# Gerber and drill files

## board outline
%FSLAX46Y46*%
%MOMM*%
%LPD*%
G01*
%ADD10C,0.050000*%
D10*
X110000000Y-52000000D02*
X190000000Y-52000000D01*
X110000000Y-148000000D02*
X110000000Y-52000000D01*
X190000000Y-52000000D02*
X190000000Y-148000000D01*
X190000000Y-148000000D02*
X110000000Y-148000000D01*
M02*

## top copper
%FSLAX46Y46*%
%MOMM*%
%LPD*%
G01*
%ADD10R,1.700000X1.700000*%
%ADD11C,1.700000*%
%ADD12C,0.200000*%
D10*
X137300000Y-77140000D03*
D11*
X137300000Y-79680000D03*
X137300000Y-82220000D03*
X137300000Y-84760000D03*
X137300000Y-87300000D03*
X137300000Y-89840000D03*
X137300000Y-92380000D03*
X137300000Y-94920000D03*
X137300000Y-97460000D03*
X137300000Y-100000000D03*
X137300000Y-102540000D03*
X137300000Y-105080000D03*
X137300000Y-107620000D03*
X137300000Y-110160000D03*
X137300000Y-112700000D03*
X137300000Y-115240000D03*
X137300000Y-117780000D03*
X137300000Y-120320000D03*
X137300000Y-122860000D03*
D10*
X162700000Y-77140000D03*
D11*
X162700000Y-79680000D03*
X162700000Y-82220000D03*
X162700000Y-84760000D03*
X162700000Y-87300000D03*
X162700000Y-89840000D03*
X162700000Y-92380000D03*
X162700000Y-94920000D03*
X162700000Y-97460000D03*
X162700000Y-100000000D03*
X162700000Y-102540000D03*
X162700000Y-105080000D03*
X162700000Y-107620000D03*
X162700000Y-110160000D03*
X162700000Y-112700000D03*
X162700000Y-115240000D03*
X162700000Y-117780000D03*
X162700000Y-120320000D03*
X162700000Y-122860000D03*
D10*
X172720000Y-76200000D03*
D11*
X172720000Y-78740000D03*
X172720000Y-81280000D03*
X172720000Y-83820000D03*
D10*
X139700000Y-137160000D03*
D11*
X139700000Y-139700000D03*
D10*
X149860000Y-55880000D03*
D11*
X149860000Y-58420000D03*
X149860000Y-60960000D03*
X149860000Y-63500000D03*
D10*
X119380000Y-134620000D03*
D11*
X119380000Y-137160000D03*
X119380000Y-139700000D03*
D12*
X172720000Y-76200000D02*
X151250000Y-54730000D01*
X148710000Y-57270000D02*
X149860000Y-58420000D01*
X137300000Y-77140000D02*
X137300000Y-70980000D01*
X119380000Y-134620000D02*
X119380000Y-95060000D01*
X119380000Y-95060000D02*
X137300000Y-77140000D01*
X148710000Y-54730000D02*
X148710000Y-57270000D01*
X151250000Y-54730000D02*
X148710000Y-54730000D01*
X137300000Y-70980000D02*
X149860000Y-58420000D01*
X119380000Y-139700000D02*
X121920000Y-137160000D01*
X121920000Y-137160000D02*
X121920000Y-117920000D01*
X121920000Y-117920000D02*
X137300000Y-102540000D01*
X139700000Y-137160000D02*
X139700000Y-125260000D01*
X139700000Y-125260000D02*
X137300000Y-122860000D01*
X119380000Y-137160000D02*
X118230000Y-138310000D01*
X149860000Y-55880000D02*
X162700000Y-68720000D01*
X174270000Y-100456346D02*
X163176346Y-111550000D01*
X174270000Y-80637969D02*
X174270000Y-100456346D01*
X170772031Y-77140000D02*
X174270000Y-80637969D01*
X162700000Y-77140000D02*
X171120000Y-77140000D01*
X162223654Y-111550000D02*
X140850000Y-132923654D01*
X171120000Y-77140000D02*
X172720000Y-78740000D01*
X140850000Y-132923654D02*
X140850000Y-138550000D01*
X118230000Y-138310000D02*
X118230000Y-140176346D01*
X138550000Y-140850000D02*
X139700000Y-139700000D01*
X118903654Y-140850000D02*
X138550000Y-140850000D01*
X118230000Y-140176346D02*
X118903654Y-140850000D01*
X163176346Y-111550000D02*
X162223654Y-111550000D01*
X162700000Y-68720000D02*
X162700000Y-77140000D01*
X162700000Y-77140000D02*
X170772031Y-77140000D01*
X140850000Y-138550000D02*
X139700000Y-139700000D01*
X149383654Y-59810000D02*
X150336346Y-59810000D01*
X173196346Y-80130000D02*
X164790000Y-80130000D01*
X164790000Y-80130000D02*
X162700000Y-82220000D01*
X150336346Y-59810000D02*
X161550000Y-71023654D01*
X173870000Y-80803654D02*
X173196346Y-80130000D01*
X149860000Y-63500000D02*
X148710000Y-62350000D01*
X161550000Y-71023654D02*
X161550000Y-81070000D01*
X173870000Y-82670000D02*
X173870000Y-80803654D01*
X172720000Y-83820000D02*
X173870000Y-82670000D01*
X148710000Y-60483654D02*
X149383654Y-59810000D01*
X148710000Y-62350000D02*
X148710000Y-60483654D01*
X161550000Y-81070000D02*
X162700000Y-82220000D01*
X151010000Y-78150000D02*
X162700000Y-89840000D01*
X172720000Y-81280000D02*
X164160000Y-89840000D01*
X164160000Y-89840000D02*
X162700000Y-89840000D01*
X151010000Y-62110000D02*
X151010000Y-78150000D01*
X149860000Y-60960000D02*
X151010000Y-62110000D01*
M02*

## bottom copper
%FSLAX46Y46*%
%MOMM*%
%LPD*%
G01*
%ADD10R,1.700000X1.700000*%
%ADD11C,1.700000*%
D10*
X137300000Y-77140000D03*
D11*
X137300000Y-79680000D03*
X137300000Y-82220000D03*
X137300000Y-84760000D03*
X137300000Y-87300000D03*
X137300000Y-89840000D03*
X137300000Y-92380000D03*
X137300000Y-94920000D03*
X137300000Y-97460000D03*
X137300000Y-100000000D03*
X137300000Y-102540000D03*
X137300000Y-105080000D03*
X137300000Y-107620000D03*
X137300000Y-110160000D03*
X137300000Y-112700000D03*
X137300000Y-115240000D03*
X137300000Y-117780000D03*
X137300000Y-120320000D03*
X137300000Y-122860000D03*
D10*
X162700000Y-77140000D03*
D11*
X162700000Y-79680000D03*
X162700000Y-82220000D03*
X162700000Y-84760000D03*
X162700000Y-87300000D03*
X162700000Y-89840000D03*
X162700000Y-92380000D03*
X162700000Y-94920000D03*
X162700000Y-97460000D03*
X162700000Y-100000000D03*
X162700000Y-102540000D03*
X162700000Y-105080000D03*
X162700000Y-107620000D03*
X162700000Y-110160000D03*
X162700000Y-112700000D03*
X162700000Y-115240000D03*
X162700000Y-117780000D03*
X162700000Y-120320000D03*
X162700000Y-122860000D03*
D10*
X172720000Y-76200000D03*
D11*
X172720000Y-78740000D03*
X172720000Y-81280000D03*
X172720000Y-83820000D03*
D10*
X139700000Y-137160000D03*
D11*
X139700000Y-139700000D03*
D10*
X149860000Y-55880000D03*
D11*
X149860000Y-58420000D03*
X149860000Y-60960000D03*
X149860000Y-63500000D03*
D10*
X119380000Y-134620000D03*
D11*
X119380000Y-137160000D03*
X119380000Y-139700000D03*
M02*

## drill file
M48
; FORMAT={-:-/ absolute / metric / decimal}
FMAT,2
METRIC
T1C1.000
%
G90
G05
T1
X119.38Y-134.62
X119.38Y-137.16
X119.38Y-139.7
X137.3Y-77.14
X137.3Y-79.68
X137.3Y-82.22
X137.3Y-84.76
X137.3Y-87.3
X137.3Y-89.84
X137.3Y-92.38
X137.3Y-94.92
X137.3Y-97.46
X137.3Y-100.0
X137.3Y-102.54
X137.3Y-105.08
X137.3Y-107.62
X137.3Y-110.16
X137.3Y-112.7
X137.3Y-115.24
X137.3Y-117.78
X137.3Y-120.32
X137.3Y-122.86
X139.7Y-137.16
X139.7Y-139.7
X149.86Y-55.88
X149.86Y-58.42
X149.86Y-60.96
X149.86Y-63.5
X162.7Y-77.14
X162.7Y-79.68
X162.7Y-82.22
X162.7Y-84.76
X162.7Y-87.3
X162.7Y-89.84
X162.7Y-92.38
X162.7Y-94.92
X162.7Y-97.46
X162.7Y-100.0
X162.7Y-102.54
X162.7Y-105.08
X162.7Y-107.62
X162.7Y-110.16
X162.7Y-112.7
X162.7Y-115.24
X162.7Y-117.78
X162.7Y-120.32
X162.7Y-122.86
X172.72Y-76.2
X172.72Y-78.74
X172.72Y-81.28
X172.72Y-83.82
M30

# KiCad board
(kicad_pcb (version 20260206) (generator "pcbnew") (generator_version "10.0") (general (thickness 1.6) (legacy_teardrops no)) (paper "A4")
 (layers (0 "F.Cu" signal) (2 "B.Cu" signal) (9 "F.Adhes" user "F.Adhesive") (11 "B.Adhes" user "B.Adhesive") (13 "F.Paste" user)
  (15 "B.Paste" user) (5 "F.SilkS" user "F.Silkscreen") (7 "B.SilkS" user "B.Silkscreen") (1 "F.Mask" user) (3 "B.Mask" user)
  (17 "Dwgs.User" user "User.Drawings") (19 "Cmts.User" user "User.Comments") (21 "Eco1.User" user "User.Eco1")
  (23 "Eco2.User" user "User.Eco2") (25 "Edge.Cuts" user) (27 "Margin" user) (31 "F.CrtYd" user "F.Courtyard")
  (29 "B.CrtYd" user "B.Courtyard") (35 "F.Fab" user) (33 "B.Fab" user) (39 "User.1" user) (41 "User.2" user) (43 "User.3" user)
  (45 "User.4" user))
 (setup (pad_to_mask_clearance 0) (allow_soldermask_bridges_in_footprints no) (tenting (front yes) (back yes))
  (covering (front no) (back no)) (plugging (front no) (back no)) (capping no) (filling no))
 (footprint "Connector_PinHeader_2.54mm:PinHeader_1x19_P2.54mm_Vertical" (layer "F.Cu") (at 137.3 77.14)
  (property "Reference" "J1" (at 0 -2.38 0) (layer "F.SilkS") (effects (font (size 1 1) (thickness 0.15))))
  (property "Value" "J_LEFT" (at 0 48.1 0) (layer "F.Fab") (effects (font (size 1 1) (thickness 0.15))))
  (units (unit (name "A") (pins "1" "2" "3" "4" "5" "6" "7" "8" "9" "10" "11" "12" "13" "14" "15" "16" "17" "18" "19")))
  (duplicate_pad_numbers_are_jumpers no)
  (pad "1" thru_hole rect (at 0 0) (size 1.7 1.7) (drill 1) (layers "*.Cu" "*.Mask") (remove_unused_layers no) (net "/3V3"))
  (pad "2" thru_hole circle (at 0 2.54) (size 1.7 1.7) (drill 1) (layers "*.Cu" "*.Mask") (remove_unused_layers no)
   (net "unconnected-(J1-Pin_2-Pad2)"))
  (pad "3" thru_hole circle (at 0 5.08) (size 1.7 1.7) (drill 1) (layers "*.Cu" "*.Mask") (remove_unused_layers no)
   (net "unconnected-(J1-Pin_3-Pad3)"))
  (pad "4" thru_hole circle (at 0 7.62) (size 1.7 1.7) (drill 1) (layers "*.Cu" "*.Mask") (remove_unused_layers no)
   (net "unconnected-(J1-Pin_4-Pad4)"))
  (pad "5" thru_hole circle (at 0 10.16) (size 1.7 1.7) (drill 1) (layers "*.Cu" "*.Mask") (remove_unused_layers no)
   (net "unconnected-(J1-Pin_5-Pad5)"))
  (pad "6" thru_hole circle (at 0 12.7) (size 1.7 1.7) (drill 1) (layers "*.Cu" "*.Mask") (remove_unused_layers no)
   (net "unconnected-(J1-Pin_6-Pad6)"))
  (pad "7" thru_hole circle (at 0 15.24) (size 1.7 1.7) (drill 1) (layers "*.Cu" "*.Mask") (remove_unused_layers no)
   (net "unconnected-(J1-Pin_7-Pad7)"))
  (pad "8" thru_hole circle (at 0 17.78) (size 1.7 1.7) (drill 1) (layers "*.Cu" "*.Mask") (remove_unused_layers no)
   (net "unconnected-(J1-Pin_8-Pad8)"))
  (pad "9" thru_hole circle (at 0 20.32) (size 1.7 1.7) (drill 1) (layers "*.Cu" "*.Mask") (remove_unused_layers no)
   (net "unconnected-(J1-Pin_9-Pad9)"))
  (pad "10" thru_hole circle (at 0 22.86) (size 1.7 1.7) (drill 1) (layers "*.Cu" "*.Mask") (remove_unused_layers no)
   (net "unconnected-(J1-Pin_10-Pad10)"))
  (pad "11" thru_hole circle (at 0 25.4) (size 1.7 1.7) (drill 1) (layers "*.Cu" "*.Mask") (remove_unused_layers no) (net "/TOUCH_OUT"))
  (pad "12" thru_hole circle (at 0 27.94) (size 1.7 1.7) (drill 1) (layers "*.Cu" "*.Mask") (remove_unused_layers no)
   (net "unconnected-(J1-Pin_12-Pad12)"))
  (pad "13" thru_hole circle (at 0 30.48) (size 1.7 1.7) (drill 1) (layers "*.Cu" "*.Mask") (remove_unused_layers no)
   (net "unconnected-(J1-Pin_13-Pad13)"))
  (pad "14" thru_hole circle (at 0 33.02) (size 1.7 1.7) (drill 1) (layers "*.Cu" "*.Mask") (remove_unused_layers no)
   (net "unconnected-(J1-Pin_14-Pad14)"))
  (pad "15" thru_hole circle (at 0 35.56) (size 1.7 1.7) (drill 1) (layers "*.Cu" "*.Mask") (remove_unused_layers no)
   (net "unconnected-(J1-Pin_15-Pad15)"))
  (pad "16" thru_hole circle (at 0 38.1) (size 1.7 1.7) (drill 1) (layers "*.Cu" "*.Mask") (remove_unused_layers no)
   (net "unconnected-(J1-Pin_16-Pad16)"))
  (pad "17" thru_hole circle (at 0 40.64) (size 1.7 1.7) (drill 1) (layers "*.Cu" "*.Mask") (remove_unused_layers no)
   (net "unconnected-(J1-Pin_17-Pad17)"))
  (pad "18" thru_hole circle (at 0 43.18) (size 1.7 1.7) (drill 1) (layers "*.Cu" "*.Mask") (remove_unused_layers no)
   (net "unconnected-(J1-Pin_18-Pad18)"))
  (pad "19" thru_hole circle (at 0 45.72) (size 1.7 1.7) (drill 1) (layers "*.Cu" "*.Mask") (remove_unused_layers no) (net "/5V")))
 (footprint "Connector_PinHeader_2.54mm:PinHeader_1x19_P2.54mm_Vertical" (layer "F.Cu") (at 162.7 77.14)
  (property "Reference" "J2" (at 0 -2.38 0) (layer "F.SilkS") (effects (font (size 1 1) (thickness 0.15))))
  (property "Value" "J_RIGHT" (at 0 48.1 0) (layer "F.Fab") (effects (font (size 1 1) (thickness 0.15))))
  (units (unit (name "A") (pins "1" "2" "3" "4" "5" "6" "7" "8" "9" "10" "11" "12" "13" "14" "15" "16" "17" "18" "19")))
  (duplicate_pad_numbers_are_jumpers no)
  (pad "1" thru_hole rect (at 0 0) (size 1.7 1.7) (drill 1) (layers "*.Cu" "*.Mask") (remove_unused_layers no) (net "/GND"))
  (pad "2" thru_hole circle (at 0 2.54) (size 1.7 1.7) (drill 1) (layers "*.Cu" "*.Mask") (remove_unused_layers no)
   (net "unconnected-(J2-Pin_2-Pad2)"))
  (pad "3" thru_hole circle (at 0 5.08) (size 1.7 1.7) (drill 1) (layers "*.Cu" "*.Mask") (remove_unused_layers no) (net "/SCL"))
  (pad "4" thru_hole circle (at 0 7.62) (size 1.7 1.7) (drill 1) (layers "*.Cu" "*.Mask") (remove_unused_layers no)
   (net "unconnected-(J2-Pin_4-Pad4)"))
  (pad "5" thru_hole circle (at 0 10.16) (size 1.7 1.7) (drill 1) (layers "*.Cu" "*.Mask") (remove_unused_layers no)
   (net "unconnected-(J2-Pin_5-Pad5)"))
  (pad "6" thru_hole circle (at 0 12.7) (size 1.7 1.7) (drill 1) (layers "*.Cu" "*.Mask") (remove_unused_layers no) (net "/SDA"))
  (pad "7" thru_hole circle (at 0 15.24) (size 1.7 1.7) (drill 1) (layers "*.Cu" "*.Mask") (remove_unused_layers no)
   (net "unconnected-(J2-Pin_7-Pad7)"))
  (pad "8" thru_hole circle (at 0 17.78) (size 1.7 1.7) (drill 1) (layers "*.Cu" "*.Mask") (remove_unused_layers no)
   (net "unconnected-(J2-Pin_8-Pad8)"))
  (pad "9" thru_hole circle (at 0 20.32) (size 1.7 1.7) (drill 1) (layers "*.Cu" "*.Mask") (remove_unused_layers no)
   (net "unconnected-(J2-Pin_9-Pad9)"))
  (pad "10" thru_hole circle (at 0 22.86) (size 1.7 1.7) (drill 1) (layers "*.Cu" "*.Mask") (remove_unused_layers no)
   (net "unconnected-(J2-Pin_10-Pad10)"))
  (pad "11" thru_hole circle (at 0 25.4) (size 1.7 1.7) (drill 1) (layers "*.Cu" "*.Mask") (remove_unused_layers no)
   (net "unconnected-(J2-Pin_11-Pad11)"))
  (pad "12" thru_hole circle (at 0 27.94) (size 1.7 1.7) (drill 1) (layers "*.Cu" "*.Mask") (remove_unused_layers no)
   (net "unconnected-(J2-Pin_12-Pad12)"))
  (pad "13" thru_hole circle (at 0 30.48) (size 1.7 1.7) (drill 1) (layers "*.Cu" "*.Mask") (remove_unused_layers no)
   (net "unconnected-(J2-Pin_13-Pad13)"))
  (pad "14" thru_hole circle (at 0 33.02) (size 1.7 1.7) (drill 1) (layers "*.Cu" "*.Mask") (remove_unused_layers no)
   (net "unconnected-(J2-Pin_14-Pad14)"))
  (pad "15" thru_hole circle (at 0 35.56) (size 1.7 1.7) (drill 1) (layers "*.Cu" "*.Mask") (remove_unused_layers no)
   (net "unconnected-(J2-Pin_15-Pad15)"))
  (pad "16" thru_hole circle (at 0 38.1) (size 1.7 1.7) (drill 1) (layers "*.Cu" "*.Mask") (remove_unused_layers no)
   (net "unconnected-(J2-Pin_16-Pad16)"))
  (pad "17" thru_hole circle (at 0 40.64) (size 1.7 1.7) (drill 1) (layers "*.Cu" "*.Mask") (remove_unused_layers no)
   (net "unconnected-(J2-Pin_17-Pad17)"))
  (pad "18" thru_hole circle (at 0 43.18) (size 1.7 1.7) (drill 1) (layers "*.Cu" "*.Mask") (remove_unused_layers no)
   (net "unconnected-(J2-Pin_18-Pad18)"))
  (pad "19" thru_hole circle (at 0 45.72) (size 1.7 1.7) (drill 1) (layers "*.Cu" "*.Mask") (remove_unused_layers no)
   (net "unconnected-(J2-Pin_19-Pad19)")))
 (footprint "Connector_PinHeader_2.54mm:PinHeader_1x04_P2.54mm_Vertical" (layer "F.Cu") (at 172.72 76.2)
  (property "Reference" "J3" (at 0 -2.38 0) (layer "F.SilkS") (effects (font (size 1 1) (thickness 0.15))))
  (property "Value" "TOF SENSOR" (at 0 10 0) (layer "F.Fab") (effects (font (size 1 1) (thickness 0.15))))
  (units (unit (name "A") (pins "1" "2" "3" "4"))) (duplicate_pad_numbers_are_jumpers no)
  (pad "1" thru_hole rect (at 0 0) (size 1.7 1.7) (drill 1) (layers "*.Cu" "*.Mask") (remove_unused_layers no) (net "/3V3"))
  (pad "2" thru_hole circle (at 0 2.54) (size 1.7 1.7) (drill 1) (layers "*.Cu" "*.Mask") (remove_unused_layers no) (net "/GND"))
  (pad "3" thru_hole circle (at 0 5.08) (size 1.7 1.7) (drill 1) (layers "*.Cu" "*.Mask") (remove_unused_layers no) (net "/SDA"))
  (pad "4" thru_hole circle (at 0 7.62) (size 1.7 1.7) (drill 1) (layers "*.Cu" "*.Mask") (remove_unused_layers no) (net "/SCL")))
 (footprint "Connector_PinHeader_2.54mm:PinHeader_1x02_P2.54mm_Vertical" (layer "F.Cu") (at 139.7 137.16)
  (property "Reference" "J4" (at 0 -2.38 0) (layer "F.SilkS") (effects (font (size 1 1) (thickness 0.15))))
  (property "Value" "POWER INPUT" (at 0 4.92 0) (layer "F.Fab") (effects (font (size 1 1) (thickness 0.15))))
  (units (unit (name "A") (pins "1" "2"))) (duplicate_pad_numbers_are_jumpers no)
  (pad "1" thru_hole rect (at 0 0) (size 1.7 1.7) (drill 1) (layers "*.Cu" "*.Mask") (remove_unused_layers no) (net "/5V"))
  (pad "2" thru_hole circle (at 0 2.54) (size 1.7 1.7) (drill 1) (layers "*.Cu" "*.Mask") (remove_unused_layers no) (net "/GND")))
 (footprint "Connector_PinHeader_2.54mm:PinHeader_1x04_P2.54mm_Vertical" (layer "F.Cu") (at 149.86 55.88)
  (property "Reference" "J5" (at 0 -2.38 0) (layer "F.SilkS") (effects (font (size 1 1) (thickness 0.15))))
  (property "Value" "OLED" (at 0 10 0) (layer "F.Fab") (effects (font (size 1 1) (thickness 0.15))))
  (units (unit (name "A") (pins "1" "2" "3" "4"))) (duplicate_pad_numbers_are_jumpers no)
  (pad "1" thru_hole rect (at 0 0) (size 1.7 1.7) (drill 1) (layers "*.Cu" "*.Mask") (remove_unused_layers no) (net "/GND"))
  (pad "2" thru_hole circle (at 0 2.54) (size 1.7 1.7) (drill 1) (layers "*.Cu" "*.Mask") (remove_unused_layers no) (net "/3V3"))
  (pad "3" thru_hole circle (at 0 5.08) (size 1.7 1.7) (drill 1) (layers "*.Cu" "*.Mask") (remove_unused_layers no) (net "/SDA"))
  (pad "4" thru_hole circle (at 0 7.62) (size 1.7 1.7) (drill 1) (layers "*.Cu" "*.Mask") (remove_unused_layers no) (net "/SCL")))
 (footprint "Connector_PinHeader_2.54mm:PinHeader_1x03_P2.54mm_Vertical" (layer "F.Cu") (at 119.38 134.62)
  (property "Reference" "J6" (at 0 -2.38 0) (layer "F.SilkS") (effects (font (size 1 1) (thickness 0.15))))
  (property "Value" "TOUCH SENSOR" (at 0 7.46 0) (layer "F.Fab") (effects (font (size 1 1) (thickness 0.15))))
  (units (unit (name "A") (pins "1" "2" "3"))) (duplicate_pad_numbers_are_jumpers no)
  (pad "1" thru_hole rect (at 0 0) (size 1.7 1.7) (drill 1) (layers "*.Cu" "*.Mask") (remove_unused_layers no) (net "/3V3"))
  (pad "2" thru_hole circle (at 0 2.54) (size 1.7 1.7) (drill 1) (layers "*.Cu" "*.Mask") (remove_unused_layers no) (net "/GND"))
  (pad "3" thru_hole circle (at 0 5.08) (size 1.7 1.7) (drill 1) (layers "*.Cu" "*.Mask") (remove_unused_layers no) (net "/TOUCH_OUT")))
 (gr_line (start 110 52) (end 190 52) (stroke (width 0.05) (type solid)) (layer "Edge.Cuts"))
 (gr_line (start 110 148) (end 110 52) (stroke (width 0.05) (type solid)) (layer "Edge.Cuts"))
 (gr_line (start 190 52) (end 190 148) (stroke (width 0.05) (type solid)) (layer "Edge.Cuts"))
 (gr_line (start 190 148) (end 110 148) (stroke (width 0.05) (type solid)) (layer "Edge.Cuts"))
 (segment (start 172.72 76.2) (end 151.25 54.73) (width 0.2) (layer "F.Cu") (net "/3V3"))
 (segment (start 148.71 57.27) (end 149.86 58.42) (width 0.2) (layer "F.Cu") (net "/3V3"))
 (segment (start 137.3 77.14) (end 137.3 70.98) (width 0.2) (layer "F.Cu") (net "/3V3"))
 (segment (start 119.38 134.62) (end 119.38 95.06) (width 0.2) (layer "F.Cu") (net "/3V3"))
 (segment (start 119.38 95.06) (end 137.3 77.14) (width 0.2) (layer "F.Cu") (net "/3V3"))
 (segment (start 148.71 54.73) (end 148.71 57.27) (width 0.2) (layer "F.Cu") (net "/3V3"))
 (segment (start 151.25 54.73) (end 148.71 54.73) (width 0.2) (layer "F.Cu") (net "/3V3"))
 (segment (start 137.3 70.98) (end 149.86 58.42) (width 0.2) (layer "F.Cu") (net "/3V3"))
 (segment (start 119.38 139.7) (end 121.92 137.16) (width 0.2) (layer "F.Cu") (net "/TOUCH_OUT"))
 (segment (start 121.92 137.16) (end 121.92 117.92) (width 0.2) (layer "F.Cu") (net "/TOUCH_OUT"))
 (segment (start 121.92 117.92) (end 137.3 102.54) (width 0.2) (layer "F.Cu") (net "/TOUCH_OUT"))
 (segment (start 139.7 137.16) (end 139.7 125.26) (width 0.2) (layer "F.Cu") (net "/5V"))
 (segment (start 139.7 125.26) (end 137.3 122.86) (width 0.2) (layer "F.Cu") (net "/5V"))
 (segment (start 119.38 137.16) (end 118.23 138.31) (width 0.2) (layer "F.Cu") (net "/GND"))
 (segment (start 149.86 55.88) (end 162.7 68.72) (width 0.2) (layer "F.Cu") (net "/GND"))
 (segment (start 174.27 100.456346) (end 163.176346 111.55) (width 0.2) (layer "F.Cu") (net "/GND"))
 (segment (start 174.27 80.637969) (end 174.27 100.456346) (width 0.2) (layer "F.Cu") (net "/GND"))
 (segment (start 170.772031 77.14) (end 174.27 80.637969) (width 0.2) (layer "F.Cu") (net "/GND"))
 (segment (start 162.7 77.14) (end 171.12 77.14) (width 0.2) (layer "F.Cu") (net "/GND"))
 (segment (start 162.223654 111.55) (end 140.85 132.923654) (width 0.2) (layer "F.Cu") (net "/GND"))
 (segment (start 171.12 77.14) (end 172.72 78.74) (width 0.2) (layer "F.Cu") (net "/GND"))
 (segment (start 140.85 132.923654) (end 140.85 138.55) (width 0.2) (layer "F.Cu") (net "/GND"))
 (segment (start 118.23 138.31) (end 118.23 140.176346) (width 0.2) (layer "F.Cu") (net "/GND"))
 (segment (start 138.55 140.85) (end 139.7 139.7) (width 0.2) (layer "F.Cu") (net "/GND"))
 (segment (start 118.903654 140.85) (end 138.55 140.85) (width 0.2) (layer "F.Cu") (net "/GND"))
 (segment (start 118.23 140.176346) (end 118.903654 140.85) (width 0.2) (layer "F.Cu") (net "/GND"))
 (segment (start 163.176346 111.55) (end 162.223654 111.55) (width 0.2) (layer "F.Cu") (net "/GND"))
 (segment (start 162.7 68.72) (end 162.7 77.14) (width 0.2) (layer "F.Cu") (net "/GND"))
 (segment (start 162.7 77.14) (end 170.772031 77.14) (width 0.2) (layer "F.Cu") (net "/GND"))
 (segment (start 140.85 138.55) (end 139.7 139.7) (width 0.2) (layer "F.Cu") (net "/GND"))
 (segment (start 149.383654 59.81) (end 150.336346 59.81) (width 0.2) (layer "F.Cu") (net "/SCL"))
 (segment (start 173.196346 80.13) (end 164.79 80.13) (width 0.2) (layer "F.Cu") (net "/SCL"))
 (segment (start 164.79 80.13) (end 162.7 82.22) (width 0.2) (layer "F.Cu") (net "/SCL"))
 (segment (start 150.336346 59.81) (end 161.55 71.023654) (width 0.2) (layer "F.Cu") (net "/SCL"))
 (segment (start 173.87 80.803654) (end 173.196346 80.13) (width 0.2) (layer "F.Cu") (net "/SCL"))
 (segment (start 149.86 63.5) (end 148.71 62.35) (width 0.2) (layer "F.Cu") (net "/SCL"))
 (segment (start 161.55 71.023654) (end 161.55 81.07) (width 0.2) (layer "F.Cu") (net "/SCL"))
 (segment (start 173.87 82.67) (end 173.87 80.803654) (width 0.2) (layer "F.Cu") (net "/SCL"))
 (segment (start 172.72 83.82) (end 173.87 82.67) (width 0.2) (layer "F.Cu") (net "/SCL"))
 (segment (start 148.71 60.483654) (end 149.383654 59.81) (width 0.2) (layer "F.Cu") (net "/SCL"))
 (segment (start 148.71 62.35) (end 148.71 60.483654) (width 0.2) (layer "F.Cu") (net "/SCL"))
 (segment (start 161.55 81.07) (end 162.7 82.22) (width 0.2) (layer "F.Cu") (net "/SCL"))
 (segment (start 151.01 78.15) (end 162.7 89.84) (width 0.2) (layer "F.Cu") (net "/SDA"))
 (segment (start 172.72 81.28) (end 164.16 89.84) (width 0.2) (layer "F.Cu") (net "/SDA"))
 (segment (start 164.16 89.84) (end 162.7 89.84) (width 0.2) (layer "F.Cu") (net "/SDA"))
 (segment (start 151.01 62.11) (end 151.01 78.15) (width 0.2) (layer "F.Cu") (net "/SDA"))
 (segment (start 149.86 60.96) (end 151.01 62.11) (width 0.2) (layer "F.Cu") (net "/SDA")))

